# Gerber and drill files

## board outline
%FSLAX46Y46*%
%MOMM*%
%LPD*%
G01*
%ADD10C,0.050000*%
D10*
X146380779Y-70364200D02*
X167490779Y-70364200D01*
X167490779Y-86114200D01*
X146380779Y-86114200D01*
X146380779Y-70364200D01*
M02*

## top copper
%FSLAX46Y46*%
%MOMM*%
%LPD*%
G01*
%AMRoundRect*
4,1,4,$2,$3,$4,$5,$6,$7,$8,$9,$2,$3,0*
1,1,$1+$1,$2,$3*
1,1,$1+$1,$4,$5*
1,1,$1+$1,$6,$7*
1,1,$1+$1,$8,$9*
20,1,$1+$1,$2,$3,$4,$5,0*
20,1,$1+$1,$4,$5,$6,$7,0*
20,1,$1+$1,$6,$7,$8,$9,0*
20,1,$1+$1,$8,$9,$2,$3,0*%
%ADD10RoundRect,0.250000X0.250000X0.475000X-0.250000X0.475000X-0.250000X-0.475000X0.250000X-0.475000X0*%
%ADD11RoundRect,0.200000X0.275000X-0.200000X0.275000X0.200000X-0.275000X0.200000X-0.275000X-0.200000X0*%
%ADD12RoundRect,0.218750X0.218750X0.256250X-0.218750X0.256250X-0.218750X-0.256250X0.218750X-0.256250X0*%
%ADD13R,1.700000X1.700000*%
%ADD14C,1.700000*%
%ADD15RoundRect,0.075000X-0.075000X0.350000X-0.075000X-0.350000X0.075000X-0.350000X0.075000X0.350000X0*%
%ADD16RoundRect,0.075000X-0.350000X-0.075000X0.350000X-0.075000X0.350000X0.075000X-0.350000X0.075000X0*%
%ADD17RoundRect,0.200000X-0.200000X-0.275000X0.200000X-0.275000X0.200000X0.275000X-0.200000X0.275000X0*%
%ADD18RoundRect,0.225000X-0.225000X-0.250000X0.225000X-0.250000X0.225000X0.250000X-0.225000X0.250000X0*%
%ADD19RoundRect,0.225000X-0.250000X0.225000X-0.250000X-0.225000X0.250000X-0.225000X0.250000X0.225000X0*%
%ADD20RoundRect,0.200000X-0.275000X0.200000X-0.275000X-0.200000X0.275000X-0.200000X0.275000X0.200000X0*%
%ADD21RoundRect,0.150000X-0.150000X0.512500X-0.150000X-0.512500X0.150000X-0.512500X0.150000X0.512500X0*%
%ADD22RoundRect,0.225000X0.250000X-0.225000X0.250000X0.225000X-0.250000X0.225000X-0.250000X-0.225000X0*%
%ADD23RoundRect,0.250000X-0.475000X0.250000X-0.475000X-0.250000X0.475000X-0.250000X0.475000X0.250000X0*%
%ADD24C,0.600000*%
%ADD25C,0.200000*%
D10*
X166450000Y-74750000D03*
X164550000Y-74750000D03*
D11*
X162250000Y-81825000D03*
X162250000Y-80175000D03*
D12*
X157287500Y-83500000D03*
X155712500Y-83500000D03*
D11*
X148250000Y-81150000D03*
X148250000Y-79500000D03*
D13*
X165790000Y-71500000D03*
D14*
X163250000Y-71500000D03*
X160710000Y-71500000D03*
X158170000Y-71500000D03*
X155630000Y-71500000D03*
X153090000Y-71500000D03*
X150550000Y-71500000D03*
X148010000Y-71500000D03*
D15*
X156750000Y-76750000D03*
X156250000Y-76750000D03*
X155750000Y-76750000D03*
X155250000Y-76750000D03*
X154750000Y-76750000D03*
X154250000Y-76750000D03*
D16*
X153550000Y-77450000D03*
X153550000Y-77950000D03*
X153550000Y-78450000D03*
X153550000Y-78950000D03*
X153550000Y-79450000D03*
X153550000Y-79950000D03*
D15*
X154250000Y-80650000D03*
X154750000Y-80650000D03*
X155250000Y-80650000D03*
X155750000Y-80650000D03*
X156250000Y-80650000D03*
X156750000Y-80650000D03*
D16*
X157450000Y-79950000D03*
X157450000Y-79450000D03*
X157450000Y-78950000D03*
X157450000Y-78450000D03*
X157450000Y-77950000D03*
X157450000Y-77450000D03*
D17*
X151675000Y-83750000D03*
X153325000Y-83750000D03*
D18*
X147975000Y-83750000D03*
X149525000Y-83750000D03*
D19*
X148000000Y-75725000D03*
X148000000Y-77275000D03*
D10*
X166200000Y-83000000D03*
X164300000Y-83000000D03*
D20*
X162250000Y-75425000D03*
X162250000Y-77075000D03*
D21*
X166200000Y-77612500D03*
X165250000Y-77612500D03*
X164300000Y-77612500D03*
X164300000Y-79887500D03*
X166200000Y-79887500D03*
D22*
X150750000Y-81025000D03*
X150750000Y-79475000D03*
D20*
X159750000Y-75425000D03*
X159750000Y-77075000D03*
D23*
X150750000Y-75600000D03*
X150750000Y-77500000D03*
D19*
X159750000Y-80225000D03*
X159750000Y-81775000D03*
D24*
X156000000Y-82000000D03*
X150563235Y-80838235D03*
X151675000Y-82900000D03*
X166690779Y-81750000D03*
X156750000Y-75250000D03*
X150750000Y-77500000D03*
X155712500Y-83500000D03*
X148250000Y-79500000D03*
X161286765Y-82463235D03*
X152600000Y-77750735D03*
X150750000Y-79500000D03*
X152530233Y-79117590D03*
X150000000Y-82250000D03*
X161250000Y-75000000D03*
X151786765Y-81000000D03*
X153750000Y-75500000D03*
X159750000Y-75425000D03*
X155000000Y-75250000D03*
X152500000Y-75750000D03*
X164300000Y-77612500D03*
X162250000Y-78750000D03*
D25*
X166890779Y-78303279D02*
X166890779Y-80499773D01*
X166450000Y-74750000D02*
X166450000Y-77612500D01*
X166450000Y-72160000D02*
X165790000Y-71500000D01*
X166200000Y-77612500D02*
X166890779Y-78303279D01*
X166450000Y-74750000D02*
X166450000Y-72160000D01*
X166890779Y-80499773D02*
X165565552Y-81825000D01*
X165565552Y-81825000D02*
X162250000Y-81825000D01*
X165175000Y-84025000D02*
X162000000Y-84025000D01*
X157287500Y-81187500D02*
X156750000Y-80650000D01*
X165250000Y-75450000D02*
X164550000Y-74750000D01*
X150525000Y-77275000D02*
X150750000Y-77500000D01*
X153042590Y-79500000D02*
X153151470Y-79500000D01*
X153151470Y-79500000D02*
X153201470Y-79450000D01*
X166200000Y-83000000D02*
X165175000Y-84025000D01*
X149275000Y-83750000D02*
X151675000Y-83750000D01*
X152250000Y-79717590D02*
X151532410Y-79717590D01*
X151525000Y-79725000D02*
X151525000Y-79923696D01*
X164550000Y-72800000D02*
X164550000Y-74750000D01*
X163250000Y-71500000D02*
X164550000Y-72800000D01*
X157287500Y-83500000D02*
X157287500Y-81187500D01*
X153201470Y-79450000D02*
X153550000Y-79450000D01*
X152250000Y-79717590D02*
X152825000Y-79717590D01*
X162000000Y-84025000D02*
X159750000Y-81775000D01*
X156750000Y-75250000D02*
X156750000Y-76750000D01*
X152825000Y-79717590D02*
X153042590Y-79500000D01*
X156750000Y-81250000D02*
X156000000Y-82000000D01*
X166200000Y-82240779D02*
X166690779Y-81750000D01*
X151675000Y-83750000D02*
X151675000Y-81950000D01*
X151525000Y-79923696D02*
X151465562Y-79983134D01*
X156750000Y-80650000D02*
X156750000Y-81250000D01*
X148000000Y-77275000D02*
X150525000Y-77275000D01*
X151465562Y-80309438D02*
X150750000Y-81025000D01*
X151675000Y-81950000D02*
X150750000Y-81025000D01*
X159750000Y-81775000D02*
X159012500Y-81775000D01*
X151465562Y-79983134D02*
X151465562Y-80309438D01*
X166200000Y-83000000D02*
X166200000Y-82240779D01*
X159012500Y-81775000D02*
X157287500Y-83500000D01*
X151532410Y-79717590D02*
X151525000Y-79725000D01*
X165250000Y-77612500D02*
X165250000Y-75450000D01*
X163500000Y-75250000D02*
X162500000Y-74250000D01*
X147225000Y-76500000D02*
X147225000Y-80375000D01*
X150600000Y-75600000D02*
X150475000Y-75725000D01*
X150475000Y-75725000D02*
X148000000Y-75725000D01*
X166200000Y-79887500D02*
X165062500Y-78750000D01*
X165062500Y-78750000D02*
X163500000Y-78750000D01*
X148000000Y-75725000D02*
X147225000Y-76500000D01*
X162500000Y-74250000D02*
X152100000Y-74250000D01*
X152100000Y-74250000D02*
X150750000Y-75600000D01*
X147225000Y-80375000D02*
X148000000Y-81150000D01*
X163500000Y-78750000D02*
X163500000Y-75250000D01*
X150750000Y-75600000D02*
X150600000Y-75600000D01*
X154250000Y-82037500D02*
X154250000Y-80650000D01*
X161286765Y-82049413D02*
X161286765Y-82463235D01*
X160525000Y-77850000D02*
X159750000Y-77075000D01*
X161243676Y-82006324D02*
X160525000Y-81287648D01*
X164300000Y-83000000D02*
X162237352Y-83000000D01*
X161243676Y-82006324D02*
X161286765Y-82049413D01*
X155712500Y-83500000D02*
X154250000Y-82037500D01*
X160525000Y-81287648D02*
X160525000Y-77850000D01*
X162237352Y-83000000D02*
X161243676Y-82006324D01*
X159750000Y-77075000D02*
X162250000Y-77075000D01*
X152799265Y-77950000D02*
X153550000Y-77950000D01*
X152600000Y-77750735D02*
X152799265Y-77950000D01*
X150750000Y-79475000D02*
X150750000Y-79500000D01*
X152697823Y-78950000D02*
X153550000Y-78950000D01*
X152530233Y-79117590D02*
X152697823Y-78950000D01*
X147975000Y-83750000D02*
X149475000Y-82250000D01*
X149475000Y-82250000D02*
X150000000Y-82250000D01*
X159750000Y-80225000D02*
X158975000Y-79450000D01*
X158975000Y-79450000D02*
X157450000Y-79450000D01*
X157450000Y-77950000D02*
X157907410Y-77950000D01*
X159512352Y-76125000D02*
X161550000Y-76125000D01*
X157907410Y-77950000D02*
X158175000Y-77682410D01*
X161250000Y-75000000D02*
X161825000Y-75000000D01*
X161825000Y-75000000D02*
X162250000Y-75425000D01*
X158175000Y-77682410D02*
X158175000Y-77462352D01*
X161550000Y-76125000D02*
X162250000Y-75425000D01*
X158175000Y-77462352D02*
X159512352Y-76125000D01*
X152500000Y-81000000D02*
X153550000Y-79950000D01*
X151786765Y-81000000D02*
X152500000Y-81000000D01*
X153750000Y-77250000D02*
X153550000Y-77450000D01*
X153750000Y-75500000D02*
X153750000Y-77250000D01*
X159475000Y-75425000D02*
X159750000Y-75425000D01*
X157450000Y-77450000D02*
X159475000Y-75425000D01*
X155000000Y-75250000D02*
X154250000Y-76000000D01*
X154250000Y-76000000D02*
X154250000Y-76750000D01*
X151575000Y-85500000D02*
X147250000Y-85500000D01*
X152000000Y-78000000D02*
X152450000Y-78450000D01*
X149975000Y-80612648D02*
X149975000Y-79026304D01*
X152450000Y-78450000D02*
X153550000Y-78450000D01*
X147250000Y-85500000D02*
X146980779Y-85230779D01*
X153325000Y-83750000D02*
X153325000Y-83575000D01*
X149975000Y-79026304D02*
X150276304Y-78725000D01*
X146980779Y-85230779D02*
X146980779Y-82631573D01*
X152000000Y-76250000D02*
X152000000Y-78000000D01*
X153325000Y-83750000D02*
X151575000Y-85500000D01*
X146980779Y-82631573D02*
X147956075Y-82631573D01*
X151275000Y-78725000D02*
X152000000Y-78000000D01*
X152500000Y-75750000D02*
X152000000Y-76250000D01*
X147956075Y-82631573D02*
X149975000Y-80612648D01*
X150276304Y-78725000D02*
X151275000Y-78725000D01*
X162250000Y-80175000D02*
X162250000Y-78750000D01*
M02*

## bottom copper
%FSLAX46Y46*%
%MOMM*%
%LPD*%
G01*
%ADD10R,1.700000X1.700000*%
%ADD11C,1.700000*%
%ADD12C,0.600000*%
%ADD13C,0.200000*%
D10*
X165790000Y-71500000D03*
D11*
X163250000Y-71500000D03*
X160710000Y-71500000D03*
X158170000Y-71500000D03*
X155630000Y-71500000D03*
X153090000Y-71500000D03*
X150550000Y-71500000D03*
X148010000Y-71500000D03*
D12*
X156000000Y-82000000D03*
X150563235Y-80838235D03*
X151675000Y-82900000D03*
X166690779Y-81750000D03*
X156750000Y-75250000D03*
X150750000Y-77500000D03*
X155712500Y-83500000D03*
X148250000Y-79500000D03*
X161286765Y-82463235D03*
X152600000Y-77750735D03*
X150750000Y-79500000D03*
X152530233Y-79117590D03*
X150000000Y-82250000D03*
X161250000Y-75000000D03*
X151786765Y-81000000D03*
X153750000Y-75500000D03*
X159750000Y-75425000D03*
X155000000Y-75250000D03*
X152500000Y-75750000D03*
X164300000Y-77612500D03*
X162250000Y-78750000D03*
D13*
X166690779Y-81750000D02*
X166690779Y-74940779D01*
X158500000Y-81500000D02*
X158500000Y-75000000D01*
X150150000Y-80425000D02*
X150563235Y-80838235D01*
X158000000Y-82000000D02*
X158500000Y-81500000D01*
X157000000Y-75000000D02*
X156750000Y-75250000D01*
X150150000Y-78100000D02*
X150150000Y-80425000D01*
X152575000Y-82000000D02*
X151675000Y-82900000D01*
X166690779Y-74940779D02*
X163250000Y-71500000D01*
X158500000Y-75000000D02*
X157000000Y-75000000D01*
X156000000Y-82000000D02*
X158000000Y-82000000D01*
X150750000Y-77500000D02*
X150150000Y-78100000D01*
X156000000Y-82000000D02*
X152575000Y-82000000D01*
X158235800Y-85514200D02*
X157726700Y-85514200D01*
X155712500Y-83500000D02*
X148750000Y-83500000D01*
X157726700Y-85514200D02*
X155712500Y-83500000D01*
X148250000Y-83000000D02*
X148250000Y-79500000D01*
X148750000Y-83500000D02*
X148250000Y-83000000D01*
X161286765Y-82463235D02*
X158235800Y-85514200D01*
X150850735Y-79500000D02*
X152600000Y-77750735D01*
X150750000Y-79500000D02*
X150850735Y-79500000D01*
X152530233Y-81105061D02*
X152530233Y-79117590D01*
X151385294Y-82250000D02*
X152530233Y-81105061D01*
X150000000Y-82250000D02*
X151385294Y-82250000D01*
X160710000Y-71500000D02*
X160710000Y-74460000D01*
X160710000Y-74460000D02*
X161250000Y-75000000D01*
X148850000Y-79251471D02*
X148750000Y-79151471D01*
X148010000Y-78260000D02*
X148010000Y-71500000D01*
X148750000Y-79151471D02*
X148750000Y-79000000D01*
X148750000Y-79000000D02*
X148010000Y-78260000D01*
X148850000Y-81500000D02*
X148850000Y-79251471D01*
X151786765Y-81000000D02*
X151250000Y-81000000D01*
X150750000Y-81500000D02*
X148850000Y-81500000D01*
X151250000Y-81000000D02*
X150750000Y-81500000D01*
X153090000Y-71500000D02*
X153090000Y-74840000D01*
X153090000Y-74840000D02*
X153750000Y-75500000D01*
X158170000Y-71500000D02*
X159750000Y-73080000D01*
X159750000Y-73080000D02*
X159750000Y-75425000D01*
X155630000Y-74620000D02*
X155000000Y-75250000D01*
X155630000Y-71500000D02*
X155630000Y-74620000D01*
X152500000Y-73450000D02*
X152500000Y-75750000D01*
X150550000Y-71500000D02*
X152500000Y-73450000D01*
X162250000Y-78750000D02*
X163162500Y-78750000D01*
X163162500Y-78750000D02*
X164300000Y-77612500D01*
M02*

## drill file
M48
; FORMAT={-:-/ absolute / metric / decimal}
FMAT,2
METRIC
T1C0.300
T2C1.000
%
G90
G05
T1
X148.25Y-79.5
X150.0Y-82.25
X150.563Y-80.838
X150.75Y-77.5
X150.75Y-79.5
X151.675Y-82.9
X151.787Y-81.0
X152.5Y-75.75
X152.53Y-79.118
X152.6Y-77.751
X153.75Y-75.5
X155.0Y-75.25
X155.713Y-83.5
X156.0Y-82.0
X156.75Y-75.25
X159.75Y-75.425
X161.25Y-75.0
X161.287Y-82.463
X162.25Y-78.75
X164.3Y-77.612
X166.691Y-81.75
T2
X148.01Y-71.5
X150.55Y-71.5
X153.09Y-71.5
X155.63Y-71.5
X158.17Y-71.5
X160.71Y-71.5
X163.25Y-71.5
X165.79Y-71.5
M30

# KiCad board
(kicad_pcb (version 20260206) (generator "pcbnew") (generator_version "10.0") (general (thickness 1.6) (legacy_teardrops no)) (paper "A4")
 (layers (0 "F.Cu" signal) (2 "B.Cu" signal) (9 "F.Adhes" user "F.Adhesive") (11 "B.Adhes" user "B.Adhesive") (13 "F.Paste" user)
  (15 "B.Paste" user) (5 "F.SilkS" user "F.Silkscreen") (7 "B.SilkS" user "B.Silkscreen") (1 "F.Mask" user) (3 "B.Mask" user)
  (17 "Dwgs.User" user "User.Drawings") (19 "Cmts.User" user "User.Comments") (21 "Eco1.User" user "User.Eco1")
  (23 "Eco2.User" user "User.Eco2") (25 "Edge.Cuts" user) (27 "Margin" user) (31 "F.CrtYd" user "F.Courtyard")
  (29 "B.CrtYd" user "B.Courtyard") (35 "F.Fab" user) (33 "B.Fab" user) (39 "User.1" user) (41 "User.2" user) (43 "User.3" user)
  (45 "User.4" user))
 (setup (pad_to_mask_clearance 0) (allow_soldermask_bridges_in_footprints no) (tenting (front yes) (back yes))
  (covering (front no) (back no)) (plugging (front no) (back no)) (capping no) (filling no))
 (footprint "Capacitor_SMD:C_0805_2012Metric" (layer "F.Cu") (at 165.5 74.75 180)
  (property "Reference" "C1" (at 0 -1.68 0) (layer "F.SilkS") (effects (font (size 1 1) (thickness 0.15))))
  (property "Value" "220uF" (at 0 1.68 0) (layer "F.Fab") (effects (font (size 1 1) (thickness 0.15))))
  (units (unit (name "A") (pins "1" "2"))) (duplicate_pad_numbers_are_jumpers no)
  (pad "1" smd roundrect (at -0.95 0 180) (size 1 1.45) (layers "F.Cu" "F.Mask" "F.Paste") (roundrect_rratio 0.25) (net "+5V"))
  (pad "2" smd roundrect (at 0.95 0 180) (size 1 1.45) (layers "F.Cu" "F.Mask" "F.Paste") (roundrect_rratio 0.25) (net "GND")))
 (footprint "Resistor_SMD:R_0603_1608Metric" (layer "F.Cu") (at 162.25 81 90)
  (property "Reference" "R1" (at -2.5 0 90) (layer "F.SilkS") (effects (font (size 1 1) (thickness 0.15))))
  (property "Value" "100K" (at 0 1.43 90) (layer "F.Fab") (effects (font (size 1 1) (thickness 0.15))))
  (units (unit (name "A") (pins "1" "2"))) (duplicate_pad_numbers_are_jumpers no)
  (pad "1" smd roundrect (at -0.825 0 90) (size 0.8 0.95) (layers "F.Cu" "F.Mask" "F.Paste") (roundrect_rratio 0.25) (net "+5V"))
  (pad "2" smd roundrect (at 0.825 0 90) (size 0.8 0.95) (layers "F.Cu" "F.Mask" "F.Paste") (roundrect_rratio 0.25) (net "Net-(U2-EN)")))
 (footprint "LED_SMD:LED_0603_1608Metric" (layer "F.Cu") (at 156.5 83.5 180)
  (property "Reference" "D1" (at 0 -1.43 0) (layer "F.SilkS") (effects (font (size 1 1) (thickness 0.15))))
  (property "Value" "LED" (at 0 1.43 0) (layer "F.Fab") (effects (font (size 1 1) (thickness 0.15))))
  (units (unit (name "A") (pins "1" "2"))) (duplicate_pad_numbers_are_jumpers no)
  (pad "1" smd roundrect (at -0.7875 0 180) (size 0.875 0.95) (layers "F.Cu" "F.Mask" "F.Paste") (roundrect_rratio 0.25) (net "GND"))
  (pad "2" smd roundrect (at 0.7875 0 180) (size 0.875 0.95) (layers "F.Cu" "F.Mask" "F.Paste") (roundrect_rratio 0.25) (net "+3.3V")))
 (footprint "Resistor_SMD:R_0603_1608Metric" (layer "F.Cu") (at 148.25 80.325 90)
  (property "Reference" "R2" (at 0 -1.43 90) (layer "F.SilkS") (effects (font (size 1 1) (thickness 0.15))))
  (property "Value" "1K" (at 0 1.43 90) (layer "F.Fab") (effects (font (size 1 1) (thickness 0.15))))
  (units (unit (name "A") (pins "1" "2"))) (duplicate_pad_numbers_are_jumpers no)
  (pad "1" smd roundrect (at -0.825 0 90) (size 0.8 0.95) (layers "F.Cu" "F.Mask" "F.Paste") (roundrect_rratio 0.25) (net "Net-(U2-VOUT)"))
  (pad "2" smd roundrect (at 0.825 0 90) (size 0.8 0.95) (layers "F.Cu" "F.Mask" "F.Paste") (roundrect_rratio 0.25) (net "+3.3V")))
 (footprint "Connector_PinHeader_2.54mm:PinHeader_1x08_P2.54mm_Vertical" (layer "F.Cu") (at 165.79 71.5 -90)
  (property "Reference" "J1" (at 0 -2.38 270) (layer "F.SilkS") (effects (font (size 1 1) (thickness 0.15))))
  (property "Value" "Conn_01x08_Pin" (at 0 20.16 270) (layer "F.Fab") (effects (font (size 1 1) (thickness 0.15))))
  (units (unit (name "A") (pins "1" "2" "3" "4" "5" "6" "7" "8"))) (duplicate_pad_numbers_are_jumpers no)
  (pad "1" thru_hole rect (at 0 0 270) (size 1.7 1.7) (drill 1) (layers "*.Cu" "*.Mask") (remove_unused_layers no) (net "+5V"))
  (pad "2" thru_hole circle (at 0 2.54 270) (size 1.7 1.7) (drill 1) (layers "*.Cu" "*.Mask") (remove_unused_layers no) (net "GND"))
  (pad "3" thru_hole circle (at 0 5.08 270) (size 1.7 1.7) (drill 1) (layers "*.Cu" "*.Mask") (remove_unused_layers no) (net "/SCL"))
  (pad "4" thru_hole circle (at 0 7.62 270) (size 1.7 1.7) (drill 1) (layers "*.Cu" "*.Mask") (remove_unused_layers no) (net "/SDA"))
  (pad "5" thru_hole circle (at 0 10.16 270) (size 1.7 1.7) (drill 1) (layers "*.Cu" "*.Mask") (remove_unused_layers no) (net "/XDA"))
  (pad "6" thru_hole circle (at 0 12.7 270) (size 1.7 1.7) (drill 1) (layers "*.Cu" "*.Mask") (remove_unused_layers no) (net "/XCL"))
  (pad "7" thru_hole circle (at 0 15.24 270) (size 1.7 1.7) (drill 1) (layers "*.Cu" "*.Mask") (remove_unused_layers no) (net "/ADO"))
  (pad "8" thru_hole circle (at 0 17.78 270) (size 1.7 1.7) (drill 1) (layers "*.Cu" "*.Mask") (remove_unused_layers no) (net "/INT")))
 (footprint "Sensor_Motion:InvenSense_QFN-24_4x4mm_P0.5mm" (layer "F.Cu") (at 155.5 78.7 -90)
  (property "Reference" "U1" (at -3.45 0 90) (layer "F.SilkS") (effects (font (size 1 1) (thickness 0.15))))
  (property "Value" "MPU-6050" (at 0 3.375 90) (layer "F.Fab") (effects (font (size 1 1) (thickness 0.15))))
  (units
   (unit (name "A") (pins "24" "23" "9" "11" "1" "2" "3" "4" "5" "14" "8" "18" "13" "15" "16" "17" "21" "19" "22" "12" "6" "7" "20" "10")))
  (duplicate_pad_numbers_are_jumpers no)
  (pad "1" smd roundrect (at -1.95 -1.25 270) (size 0.85 0.3) (layers "F.Cu" "F.Mask" "F.Paste") (roundrect_rratio 0.25) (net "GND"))
  (pad "2" smd roundrect (at -1.95 -0.75 270) (size 0.85 0.3) (layers "F.Cu" "F.Mask" "F.Paste") (roundrect_rratio 0.25)
   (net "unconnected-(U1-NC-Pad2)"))
  (pad "3" smd roundrect (at -1.95 -0.25 270) (size 0.85 0.3) (layers "F.Cu" "F.Mask" "F.Paste") (roundrect_rratio 0.25)
   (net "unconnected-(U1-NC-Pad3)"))
  (pad "4" smd roundrect (at -1.95 0.25 270) (size 0.85 0.3) (layers "F.Cu" "F.Mask" "F.Paste") (roundrect_rratio 0.25)
   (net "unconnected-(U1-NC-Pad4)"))
  (pad "5" smd roundrect (at -1.95 0.75 270) (size 0.85 0.3) (layers "F.Cu" "F.Mask" "F.Paste") (roundrect_rratio 0.25)
   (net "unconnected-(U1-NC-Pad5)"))
  (pad "6" smd roundrect (at -1.95 1.25 270) (size 0.85 0.3) (layers "F.Cu" "F.Mask" "F.Paste") (roundrect_rratio 0.25) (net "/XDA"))
  (pad "7" smd roundrect (at -1.25 1.95) (size 0.85 0.3) (layers "F.Cu" "F.Mask" "F.Paste") (roundrect_rratio 0.25) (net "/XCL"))
  (pad "8" smd roundrect (at -0.75 1.95) (size 0.85 0.3) (layers "F.Cu" "F.Mask" "F.Paste") (roundrect_rratio 0.25) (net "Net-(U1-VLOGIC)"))
  (pad "9" smd roundrect (at -0.25 1.95) (size 0.85 0.3) (layers "F.Cu" "F.Mask" "F.Paste") (roundrect_rratio 0.25) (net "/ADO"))
  (pad "10" smd roundrect (at 0.25 1.95) (size 0.85 0.3) (layers "F.Cu" "F.Mask" "F.Paste") (roundrect_rratio 0.25) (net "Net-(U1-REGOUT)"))
  (pad "11" smd roundrect (at 0.75 1.95) (size 0.85 0.3) (layers "F.Cu" "F.Mask" "F.Paste") (roundrect_rratio 0.25) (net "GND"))
  (pad "12" smd roundrect (at 1.25 1.95) (size 0.85 0.3) (layers "F.Cu" "F.Mask" "F.Paste") (roundrect_rratio 0.25) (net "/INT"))
  (pad "13" smd roundrect (at 1.95 1.25 270) (size 0.85 0.3) (layers "F.Cu" "F.Mask" "F.Paste") (roundrect_rratio 0.25) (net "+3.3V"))
  (pad "14" smd roundrect (at 1.95 0.75 270) (size 0.85 0.3) (layers "F.Cu" "F.Mask" "F.Paste") (roundrect_rratio 0.25)
   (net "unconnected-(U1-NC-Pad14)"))
  (pad "15" smd roundrect (at 1.95 0.25 270) (size 0.85 0.3) (layers "F.Cu" "F.Mask" "F.Paste") (roundrect_rratio 0.25)
   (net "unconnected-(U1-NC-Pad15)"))
  (pad "16" smd roundrect (at 1.95 -0.25 270) (size 0.85 0.3) (layers "F.Cu" "F.Mask" "F.Paste") (roundrect_rratio 0.25)
   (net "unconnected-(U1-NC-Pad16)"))
  (pad "17" smd roundrect (at 1.95 -0.75 270) (size 0.85 0.3) (layers "F.Cu" "F.Mask" "F.Paste") (roundrect_rratio 0.25)
   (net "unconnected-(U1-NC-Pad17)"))
  (pad "18" smd roundrect (at 1.95 -1.25 270) (size 0.85 0.3) (layers "F.Cu" "F.Mask" "F.Paste") (roundrect_rratio 0.25) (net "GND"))
  (pad "19" smd roundrect (at 1.25 -1.95) (size 0.85 0.3) (layers "F.Cu" "F.Mask" "F.Paste") (roundrect_rratio 0.25)
   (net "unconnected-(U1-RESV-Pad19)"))
  (pad "20" smd roundrect (at 0.75 -1.95) (size 0.85 0.3) (layers "F.Cu" "F.Mask" "F.Paste") (roundrect_rratio 0.25) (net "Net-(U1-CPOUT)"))
  (pad "21" smd roundrect (at 0.25 -1.95) (size 0.85 0.3) (layers "F.Cu" "F.Mask" "F.Paste") (roundrect_rratio 0.25)
   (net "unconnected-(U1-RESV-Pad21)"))
  (pad "22" smd roundrect (at -0.25 -1.95) (size 0.85 0.3) (layers "F.Cu" "F.Mask" "F.Paste") (roundrect_rratio 0.25)
   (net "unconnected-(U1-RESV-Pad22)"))
  (pad "23" smd roundrect (at -0.75 -1.95) (size 0.85 0.3) (layers "F.Cu" "F.Mask" "F.Paste") (roundrect_rratio 0.25) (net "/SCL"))
  (pad "24" smd roundrect (at -1.25 -1.95) (size 0.85 0.3) (layers "F.Cu" "F.Mask" "F.Paste") (roundrect_rratio 0.25) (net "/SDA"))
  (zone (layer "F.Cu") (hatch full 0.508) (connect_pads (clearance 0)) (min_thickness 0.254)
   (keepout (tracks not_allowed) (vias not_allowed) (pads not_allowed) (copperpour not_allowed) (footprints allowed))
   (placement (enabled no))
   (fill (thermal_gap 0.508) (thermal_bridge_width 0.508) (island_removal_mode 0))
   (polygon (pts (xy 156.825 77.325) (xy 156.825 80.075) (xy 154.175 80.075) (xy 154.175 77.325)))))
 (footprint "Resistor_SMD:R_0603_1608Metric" (layer "F.Cu") (at 152.5 83.75)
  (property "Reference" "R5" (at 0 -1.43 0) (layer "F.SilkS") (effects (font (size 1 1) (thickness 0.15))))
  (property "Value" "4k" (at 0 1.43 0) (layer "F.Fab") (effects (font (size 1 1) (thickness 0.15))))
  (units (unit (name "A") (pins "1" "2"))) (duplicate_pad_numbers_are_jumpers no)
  (pad "1" smd roundrect (at -0.825 0) (size 0.8 0.95) (layers "F.Cu" "F.Mask" "F.Paste") (roundrect_rratio 0.25) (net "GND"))
  (pad "2" smd roundrect (at 0.825 0) (size 0.8 0.95) (layers "F.Cu" "F.Mask" "F.Paste") (roundrect_rratio 0.25) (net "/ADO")))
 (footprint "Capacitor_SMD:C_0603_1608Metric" (layer "F.Cu") (at 148.75 83.75)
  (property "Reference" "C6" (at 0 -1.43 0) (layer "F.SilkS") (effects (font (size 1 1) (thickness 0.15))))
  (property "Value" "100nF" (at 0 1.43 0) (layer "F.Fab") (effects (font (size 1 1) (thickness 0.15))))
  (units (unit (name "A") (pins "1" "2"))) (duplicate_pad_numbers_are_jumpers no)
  (pad "1" smd roundrect (at -0.775 0) (size 0.9 0.95) (layers "F.Cu" "F.Mask" "F.Paste") (roundrect_rratio 0.25) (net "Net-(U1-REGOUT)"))
  (pad "2" smd roundrect (at 0.775 0) (size 0.9 0.95) (layers "F.Cu" "F.Mask" "F.Paste") (roundrect_rratio 0.25) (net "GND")))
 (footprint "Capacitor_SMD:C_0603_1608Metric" (layer "F.Cu") (at 148 76.5 -90)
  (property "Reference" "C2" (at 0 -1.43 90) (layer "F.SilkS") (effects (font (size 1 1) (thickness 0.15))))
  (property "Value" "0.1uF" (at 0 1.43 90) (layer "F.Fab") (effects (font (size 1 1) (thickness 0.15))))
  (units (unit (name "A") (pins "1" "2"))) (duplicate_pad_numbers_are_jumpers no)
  (pad "1" smd roundrect (at -0.775 0 270) (size 0.9 0.95) (layers "F.Cu" "F.Mask" "F.Paste") (roundrect_rratio 0.25) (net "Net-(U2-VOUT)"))
  (pad "2" smd roundrect (at 0.775 0 270) (size 0.9 0.95) (layers "F.Cu" "F.Mask" "F.Paste") (roundrect_rratio 0.25) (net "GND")))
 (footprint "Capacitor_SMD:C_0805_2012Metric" (layer "F.Cu") (at 165.25 83 180)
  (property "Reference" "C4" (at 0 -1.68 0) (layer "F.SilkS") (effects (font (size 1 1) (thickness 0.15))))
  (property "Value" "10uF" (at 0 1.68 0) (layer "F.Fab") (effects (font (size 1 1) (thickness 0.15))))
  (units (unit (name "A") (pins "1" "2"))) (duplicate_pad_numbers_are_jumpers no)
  (pad "1" smd roundrect (at -0.95 0 180) (size 1 1.45) (layers "F.Cu" "F.Mask" "F.Paste") (roundrect_rratio 0.25) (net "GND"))
  (pad "2" smd roundrect (at 0.95 0 180) (size 1 1.45) (layers "F.Cu" "F.Mask" "F.Paste") (roundrect_rratio 0.25) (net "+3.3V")))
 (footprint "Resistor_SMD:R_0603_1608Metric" (layer "F.Cu") (at 162.25 76.25 -90)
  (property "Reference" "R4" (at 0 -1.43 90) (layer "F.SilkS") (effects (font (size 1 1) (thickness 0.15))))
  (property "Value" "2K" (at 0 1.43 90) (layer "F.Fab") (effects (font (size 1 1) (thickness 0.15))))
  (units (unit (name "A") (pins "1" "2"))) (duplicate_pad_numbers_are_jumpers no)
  (pad "1" smd roundrect (at -0.825 0 270) (size 0.8 0.95) (layers "F.Cu" "F.Mask" "F.Paste") (roundrect_rratio 0.25) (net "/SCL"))
  (pad "2" smd roundrect (at 0.825 0 270) (size 0.8 0.95) (layers "F.Cu" "F.Mask" "F.Paste") (roundrect_rratio 0.25) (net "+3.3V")))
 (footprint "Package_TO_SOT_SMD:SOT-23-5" (layer "F.Cu") (at 165.25 78.75 -90)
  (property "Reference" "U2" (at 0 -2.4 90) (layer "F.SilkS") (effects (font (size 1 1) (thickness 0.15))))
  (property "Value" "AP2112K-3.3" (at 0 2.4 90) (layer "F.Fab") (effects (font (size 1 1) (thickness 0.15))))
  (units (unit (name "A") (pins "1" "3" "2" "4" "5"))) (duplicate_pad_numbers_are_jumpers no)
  (pad "1" smd roundrect (at -1.1375 -0.95 270) (size 1.325 0.6) (layers "F.Cu" "F.Mask" "F.Paste") (roundrect_rratio 0.25) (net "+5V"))
  (pad "2" smd roundrect (at -1.1375 0 270) (size 1.325 0.6) (layers "F.Cu" "F.Mask" "F.Paste") (roundrect_rratio 0.25) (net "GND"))
  (pad "3" smd roundrect (at -1.1375 0.95 270) (size 1.325 0.6) (layers "F.Cu" "F.Mask" "F.Paste") (roundrect_rratio 0.25)
   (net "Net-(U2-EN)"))
  (pad "4" smd roundrect (at 1.1375 0.95 270) (size 1.325 0.6) (layers "F.Cu" "F.Mask" "F.Paste") (roundrect_rratio 0.25)
   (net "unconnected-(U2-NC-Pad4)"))
  (pad "5" smd roundrect (at 1.1375 -0.95 270) (size 1.325 0.6) (layers "F.Cu" "F.Mask" "F.Paste") (roundrect_rratio 0.25)
   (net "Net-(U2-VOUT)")))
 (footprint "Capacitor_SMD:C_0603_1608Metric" (layer "F.Cu") (at 150.75 80.25 90)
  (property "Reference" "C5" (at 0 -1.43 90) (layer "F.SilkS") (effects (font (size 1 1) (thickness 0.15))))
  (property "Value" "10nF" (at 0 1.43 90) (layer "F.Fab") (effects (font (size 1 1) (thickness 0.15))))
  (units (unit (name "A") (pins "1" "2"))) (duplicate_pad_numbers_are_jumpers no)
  (pad "1" smd roundrect (at -0.775 0 90) (size 0.9 0.95) (layers "F.Cu" "F.Mask" "F.Paste") (roundrect_rratio 0.25) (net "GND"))
  (pad "2" smd roundrect (at 0.775 0 90) (size 0.9 0.95) (layers "F.Cu" "F.Mask" "F.Paste") (roundrect_rratio 0.25) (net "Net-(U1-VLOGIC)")))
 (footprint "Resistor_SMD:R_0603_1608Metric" (layer "F.Cu") (at 159.75 76.25 -90)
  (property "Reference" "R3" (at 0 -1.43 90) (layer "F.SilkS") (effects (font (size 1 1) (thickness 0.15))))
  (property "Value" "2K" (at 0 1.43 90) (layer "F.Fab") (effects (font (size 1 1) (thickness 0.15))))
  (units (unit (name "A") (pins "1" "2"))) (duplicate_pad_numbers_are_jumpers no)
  (pad "1" smd roundrect (at -0.825 0 270) (size 0.8 0.95) (layers "F.Cu" "F.Mask" "F.Paste") (roundrect_rratio 0.25) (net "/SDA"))
  (pad "2" smd roundrect (at 0.825 0 270) (size 0.8 0.95) (layers "F.Cu" "F.Mask" "F.Paste") (roundrect_rratio 0.25) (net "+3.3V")))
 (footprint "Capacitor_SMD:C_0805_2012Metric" (layer "F.Cu") (at 150.75 76.55 -90)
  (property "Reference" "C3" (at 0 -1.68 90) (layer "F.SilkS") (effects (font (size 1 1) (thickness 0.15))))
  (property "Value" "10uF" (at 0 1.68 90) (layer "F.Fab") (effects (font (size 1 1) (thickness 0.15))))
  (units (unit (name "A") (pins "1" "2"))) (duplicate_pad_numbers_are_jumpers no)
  (pad "1" smd roundrect (at -0.95 0 270) (size 1 1.45) (layers "F.Cu" "F.Mask" "F.Paste") (roundrect_rratio 0.25) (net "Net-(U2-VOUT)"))
  (pad "2" smd roundrect (at 0.95 0 270) (size 1 1.45) (layers "F.Cu" "F.Mask" "F.Paste") (roundrect_rratio 0.25) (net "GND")))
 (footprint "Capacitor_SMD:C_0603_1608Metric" (layer "F.Cu") (at 159.75 81 -90)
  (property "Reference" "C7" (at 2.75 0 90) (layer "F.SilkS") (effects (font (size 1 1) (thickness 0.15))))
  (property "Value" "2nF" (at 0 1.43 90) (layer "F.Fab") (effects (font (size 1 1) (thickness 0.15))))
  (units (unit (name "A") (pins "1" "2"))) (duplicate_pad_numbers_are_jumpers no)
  (pad "1" smd roundrect (at -0.775 0 270) (size 0.9 0.95) (layers "F.Cu" "F.Mask" "F.Paste") (roundrect_rratio 0.25) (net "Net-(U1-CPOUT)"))
  (pad "2" smd roundrect (at 0.775 0 270) (size 0.9 0.95) (layers "F.Cu" "F.Mask" "F.Paste") (roundrect_rratio 0.25) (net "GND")))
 (gr_rect (start 146.380779 70.3642) (end 167.490779 86.1142) (stroke (width 0.05) (type solid)) (fill no) (layer "Edge.Cuts"))
 (segment (start 166.890779 78.303279) (end 166.890779 80.499773) (width 0.2) (layer "F.Cu") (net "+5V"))
 (segment (start 166.45 74.75) (end 166.45 77.6125) (width 0.2) (layer "F.Cu") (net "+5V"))
 (segment (start 166.45 72.16) (end 165.79 71.5) (width 0.2) (layer "F.Cu") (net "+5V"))
 (segment (start 166.2 77.6125) (end 166.890779 78.303279) (width 0.2) (layer "F.Cu") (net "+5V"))
 (segment (start 166.45 74.75) (end 166.45 72.16) (width 0.2) (layer "F.Cu") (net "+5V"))
 (segment (start 166.890779 80.499773) (end 165.565552 81.825) (width 0.2) (layer "F.Cu") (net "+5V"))
 (segment (start 165.565552 81.825) (end 162.25 81.825) (width 0.2) (layer "F.Cu") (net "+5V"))
 (segment (start 165.175 84.025) (end 162 84.025) (width 0.2) (layer "F.Cu") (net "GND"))
 (segment (start 157.2875 81.1875) (end 156.75 80.65) (width 0.2) (layer "F.Cu") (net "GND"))
 (segment (start 165.25 75.45) (end 164.55 74.75) (width 0.2) (layer "F.Cu") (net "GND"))
 (segment (start 150.525 77.275) (end 150.75 77.5) (width 0.2) (layer "F.Cu") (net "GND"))
 (segment (start 153.04259 79.5) (end 153.15147 79.5) (width 0.2) (layer "F.Cu") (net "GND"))
 (segment (start 153.15147 79.5) (end 153.20147 79.45) (width 0.2) (layer "F.Cu") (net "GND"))
 (segment (start 166.2 83) (end 165.175 84.025) (width 0.2) (layer "F.Cu") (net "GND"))
 (segment (start 149.275 83.75) (end 151.675 83.75) (width 0.2) (layer "F.Cu") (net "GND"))
 (segment (start 152.25 79.71759) (end 151.53241 79.71759) (width 0.2) (layer "F.Cu") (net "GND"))
 (segment (start 151.525 79.725) (end 151.525 79.923696) (width 0.2) (layer "F.Cu") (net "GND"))
 (segment (start 164.55 72.8) (end 164.55 74.75) (width 0.2) (layer "F.Cu") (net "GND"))
 (segment (start 163.25 71.5) (end 164.55 72.8) (width 0.2) (layer "F.Cu") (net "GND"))
 (segment (start 157.2875 83.5) (end 157.2875 81.1875) (width 0.2) (layer "F.Cu") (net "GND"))
 (segment (start 153.20147 79.45) (end 153.55 79.45) (width 0.2) (layer "F.Cu") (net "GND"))
 (segment (start 152.25 79.71759) (end 152.825 79.71759) (width 0.2) (layer "F.Cu") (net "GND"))
 (segment (start 162 84.025) (end 159.75 81.775) (width 0.2) (layer "F.Cu") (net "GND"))
 (segment (start 156.75 75.25) (end 156.75 76.75) (width 0.2) (layer "F.Cu") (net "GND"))
 (segment (start 152.825 79.71759) (end 153.04259 79.5) (width 0.2) (layer "F.Cu") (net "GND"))
 (segment (start 156.75 81.25) (end 156 82) (width 0.2) (layer "F.Cu") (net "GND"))
 (segment (start 166.2 82.240779) (end 166.690779 81.75) (width 0.2) (layer "F.Cu") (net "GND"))
 (segment (start 151.675 83.75) (end 151.675 81.95) (width 0.2) (layer "F.Cu") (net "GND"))
 (segment (start 151.525 79.923696) (end 151.465562 79.983134) (width 0.2) (layer "F.Cu") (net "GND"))
 (segment (start 156.75 80.65) (end 156.75 81.25) (width 0.2) (layer "F.Cu") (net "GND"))
 (segment (start 148 77.275) (end 150.525 77.275) (width 0.2) (layer "F.Cu") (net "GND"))
 (segment (start 151.465562 80.309438) (end 150.75 81.025) (width 0.2) (layer "F.Cu") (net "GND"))
 (segment (start 151.675 81.95) (end 150.75 81.025) (width 0.2) (layer "F.Cu") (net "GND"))
 (segment (start 159.75 81.775) (end 159.0125 81.775) (width 0.2) (layer "F.Cu") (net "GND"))
 (segment (start 151.465562 79.983134) (end 151.465562 80.309438) (width 0.2) (layer "F.Cu") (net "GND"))
 (segment (start 166.2 83) (end 166.2 82.240779) (width 0.2) (layer "F.Cu") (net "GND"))
 (segment (start 159.0125 81.775) (end 157.2875 83.5) (width 0.2) (layer "F.Cu") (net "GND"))
 (segment (start 151.53241 79.71759) (end 151.525 79.725) (width 0.2) (layer "F.Cu") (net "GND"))
 (segment (start 165.25 77.6125) (end 165.25 75.45) (width 0.2) (layer "F.Cu") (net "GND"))
 (via (at 156 82) (size 0.6) (drill 0.3) (layers "F.Cu" "B.Cu") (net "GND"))
 (via (at 150.563235 80.838235) (size 0.6) (drill 0.3) (layers "F.Cu" "B.Cu") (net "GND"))
 (via (at 151.675 82.9) (size 0.6) (drill 0.3) (layers "F.Cu" "B.Cu") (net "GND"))
 (via (at 166.690779 81.75) (size 0.6) (drill 0.3) (layers "F.Cu" "B.Cu") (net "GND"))
 (via (at 156.75 75.25) (size 0.6) (drill 0.3) (layers "F.Cu" "B.Cu") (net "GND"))
 (via (at 150.75 77.5) (size 0.6) (drill 0.3) (layers "F.Cu" "B.Cu") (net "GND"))
 (segment (start 166.690779 81.75) (end 166.690779 74.940779) (width 0.2) (layer "B.Cu") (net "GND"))
 (segment (start 158.5 81.5) (end 158.5 75) (width 0.2) (layer "B.Cu") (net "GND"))
 (segment (start 150.15 80.425) (end 150.563235 80.838235) (width 0.2) (layer "B.Cu") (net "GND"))
 (segment (start 158 82) (end 158.5 81.5) (width 0.2) (layer "B.Cu") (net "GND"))
 (segment (start 157 75) (end 156.75 75.25) (width 0.2) (layer "B.Cu") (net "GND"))
 (segment (start 150.15 78.1) (end 150.15 80.425) (width 0.2) (layer "B.Cu") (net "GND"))
 (segment (start 152.575 82) (end 151.675 82.9) (width 0.2) (layer "B.Cu") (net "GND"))
 (segment (start 166.690779 74.940779) (end 163.25 71.5) (width 0.2) (layer "B.Cu") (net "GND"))
 (segment (start 158.5 75) (end 157 75) (width 0.2) (layer "B.Cu") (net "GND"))
 (segment (start 156 82) (end 158 82) (width 0.2) (layer "B.Cu") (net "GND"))
 (segment (start 150.75 77.5) (end 150.15 78.1) (width 0.2) (layer "B.Cu") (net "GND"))
 (segment (start 156 82) (end 152.575 82) (width 0.2) (layer "B.Cu") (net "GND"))
 (segment (start 163.5 75.25) (end 162.5 74.25) (width 0.2) (layer "F.Cu") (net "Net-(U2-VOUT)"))
 (segment (start 147.225 76.5) (end 147.225 80.375) (width 0.2) (layer "F.Cu") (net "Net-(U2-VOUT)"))
 (segment (start 150.6 75.6) (end 150.475 75.725) (width 0.2) (layer "F.Cu") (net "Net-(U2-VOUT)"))
 (segment (start 150.475 75.725) (end 148 75.725) (width 0.2) (layer "F.Cu") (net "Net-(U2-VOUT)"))
 (segment (start 166.2 79.8875) (end 165.0625 78.75) (width 0.2) (layer "F.Cu") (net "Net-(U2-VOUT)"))
 (segment (start 165.0625 78.75) (end 163.5 78.75) (width 0.2) (layer "F.Cu") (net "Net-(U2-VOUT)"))
 (segment (start 148 75.725) (end 147.225 76.5) (width 0.2) (layer "F.Cu") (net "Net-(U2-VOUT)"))
 (segment (start 162.5 74.25) (end 152.1 74.25) (width 0.2) (layer "F.Cu") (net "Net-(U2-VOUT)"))
 (segment (start 152.1 74.25) (end 150.75 75.6) (width 0.2) (layer "F.Cu") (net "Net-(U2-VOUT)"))
 (segment (start 147.225 80.375) (end 148 81.15) (width 0.2) (layer "F.Cu") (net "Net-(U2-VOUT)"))
 (segment (start 163.5 78.75) (end 163.5 75.25) (width 0.2) (layer "F.Cu") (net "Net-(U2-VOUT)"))
 (segment (start 150.75 75.6) (end 150.6 75.6) (width 0.2) (layer "F.Cu") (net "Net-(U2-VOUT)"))
 (segment (start 154.25 82.0375) (end 154.25 80.65) (width 0.2) (layer "F.Cu") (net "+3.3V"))
 (segment (start 161.286765 82.049413) (end 161.286765 82.463235) (width 0.2) (layer "F.Cu") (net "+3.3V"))
 (segment (start 160.525 77.85) (end 159.75 77.075) (width 0.2) (layer "F.Cu") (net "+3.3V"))
 (segment (start 161.243676 82.006324) (end 160.525 81.287648) (width 0.2) (layer "F.Cu") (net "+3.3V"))
 (segment (start 164.3 83) (end 162.237352 83) (width 0.2) (layer "F.Cu") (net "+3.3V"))
 (segment (start 161.243676 82.006324) (end 161.286765 82.049413) (width 0.2) (layer "F.Cu") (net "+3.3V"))
 (segment (start 155.7125 83.5) (end 154.25 82.0375) (width 0.2) (layer "F.Cu") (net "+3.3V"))
 (segment (start 160.525 81.287648) (end 160.525 77.85) (width 0.2) (layer "F.Cu") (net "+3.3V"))
 (segment (start 162.237352 83) (end 161.243676 82.006324) (width 0.2) (layer "F.Cu") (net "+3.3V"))
 (segment (start 159.75 77.075) (end 162.25 77.075) (width 0.2) (layer "F.Cu") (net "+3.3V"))
 (via (at 155.7125 83.5) (size 0.6) (drill 0.3) (layers "F.Cu" "B.Cu") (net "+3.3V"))
 (via (at 148.25 79.5) (size 0.6) (drill 0.3) (layers "F.Cu" "B.Cu") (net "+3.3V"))
 (via (at 161.286765 82.463235) (size 0.6) (drill 0.3) (layers "F.Cu" "B.Cu") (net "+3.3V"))
 (segment (start 158.2358 85.5142) (end 157.7267 85.5142) (width 0.2) (layer "B.Cu") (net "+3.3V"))
 (segment (start 155.7125 83.5) (end 148.75 83.5) (width 0.2) (layer "B.Cu") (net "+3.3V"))
 (segment (start 157.7267 85.5142) (end 155.7125 83.5) (width 0.2) (layer "B.Cu") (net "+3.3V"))
 (segment (start 148.25 83) (end 148.25 79.5) (width 0.2) (layer "B.Cu") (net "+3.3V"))
 (segment (start 148.75 83.5) (end 148.25 83) (width 0.2) (layer "B.Cu") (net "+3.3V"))
 (segment (start 161.286765 82.463235) (end 158.2358 85.5142) (width 0.2) (layer "B.Cu") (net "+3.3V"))
 (segment (start 152.799265 77.95) (end 153.55 77.95) (width 0.2) (layer "F.Cu") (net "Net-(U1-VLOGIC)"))
 (segment (start 152.6 77.750735) (end 152.799265 77.95) (width 0.2) (layer "F.Cu") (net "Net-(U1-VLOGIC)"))
 (segment (start 150.75 79.475) (end 150.75 79.5) (width 0.2) (layer "F.Cu") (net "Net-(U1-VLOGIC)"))
 (via (at 152.6 77.750735) (size 0.6) (drill 0.3) (layers "F.Cu" "B.Cu") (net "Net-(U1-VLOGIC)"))
 (via (at 150.75 79.5) (size 0.6) (drill 0.3) (layers "F.Cu" "B.Cu") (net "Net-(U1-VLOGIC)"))
 (segment (start 150.850735 79.5) (end 152.6 77.750735) (width 0.2) (layer "B.Cu") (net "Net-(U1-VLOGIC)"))
 (segment (start 150.75 79.5) (end 150.850735 79.5) (width 0.2) (layer "B.Cu") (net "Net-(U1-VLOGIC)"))
 (segment (start 152.697823 78.95) (end 153.55 78.95) (width 0.2) (layer "F.Cu") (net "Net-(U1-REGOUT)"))
 (segment (start 152.530233 79.11759) (end 152.697823 78.95) (width 0.2) (layer "F.Cu") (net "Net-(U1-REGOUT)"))
 (segment (start 147.975 83.75) (end 149.475 82.25) (width 0.2) (layer "F.Cu") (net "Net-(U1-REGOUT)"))
 (segment (start 149.475 82.25) (end 150 82.25) (width 0.2) (layer "F.Cu") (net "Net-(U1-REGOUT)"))
 (via (at 152.530233 79.11759) (size 0.6) (drill 0.3) (layers "F.Cu" "B.Cu") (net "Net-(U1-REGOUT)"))
 (via (at 150 82.25) (size 0.6) (drill 0.3) (layers "F.Cu" "B.Cu") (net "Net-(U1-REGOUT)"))
 (segment (start 152.530233 81.105061) (end 152.530233 79.11759) (width 0.2) (layer "B.Cu") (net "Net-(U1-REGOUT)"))
 (segment (start 151.385294 82.25) (end 152.530233 81.105061) (width 0.2) (layer "B.Cu") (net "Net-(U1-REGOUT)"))
 (segment (start 150 82.25) (end 151.385294 82.25) (width 0.2) (layer "B.Cu") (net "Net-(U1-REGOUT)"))
 (segment (start 159.75 80.225) (end 158.975 79.45) (width 0.2) (layer "F.Cu") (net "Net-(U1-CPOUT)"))
 (segment (start 158.975 79.45) (end 157.45 79.45) (width 0.2) (layer "F.Cu") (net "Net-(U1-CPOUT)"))
 (segment (start 157.45 77.95) (end 157.90741 77.95) (width 0.2) (layer "F.Cu") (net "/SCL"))
 (segment (start 159.512352 76.125) (end 161.55 76.125) (width 0.2) (layer "F.Cu") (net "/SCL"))
 (segment (start 157.90741 77.95) (end 158.175 77.68241) (width 0.2) (layer "F.Cu") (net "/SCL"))
 (segment (start 161.25 75) (end 161.825 75) (width 0.2) (layer "F.Cu") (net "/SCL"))
 (segment (start 161.825 75) (end 162.25 75.425) (width 0.2) (layer "F.Cu") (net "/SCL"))
 (segment (start 158.175 77.68241) (end 158.175 77.462352) (width 0.2) (layer "F.Cu") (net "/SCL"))
 (segment (start 161.55 76.125) (end 162.25 75.425) (width 0.2) (layer "F.Cu") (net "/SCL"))
 (segment (start 158.175 77.462352) (end 159.512352 76.125) (width 0.2) (layer "F.Cu") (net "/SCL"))
 (via (at 161.25 75) (size 0.6) (drill 0.3) (layers "F.Cu" "B.Cu") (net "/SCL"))
 (segment (start 160.71 71.5) (end 160.71 74.46) (width 0.2) (layer "B.Cu") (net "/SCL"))
 (segment (start 160.71 74.46) (end 161.25 75) (width 0.2) (layer "B.Cu") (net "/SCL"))
 (segment (start 152.5 81) (end 153.55 79.95) (width 0.2) (layer "F.Cu") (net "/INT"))
 (segment (start 151.786765 81) (end 152.5 81) (width 0.2) (layer "F.Cu") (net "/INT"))
 (via (at 151.786765 81) (size 0.6) (drill 0.3) (layers "F.Cu" "B.Cu") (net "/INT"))
 (segment (start 148.85 79.251471) (end 148.75 79.151471) (width 0.2) (layer "B.Cu") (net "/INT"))
 (segment (start 148.01 78.26) (end 148.01 71.5) (width 0.2) (layer "B.Cu") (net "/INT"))
 (segment (start 148.75 79.151471) (end 148.75 79) (width 0.2) (layer "B.Cu") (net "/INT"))
 (segment (start 148.75 79) (end 148.01 78.26) (width 0.2) (layer "B.Cu") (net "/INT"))
 (segment (start 148.85 81.5) (end 148.85 79.251471) (width 0.2) (layer "B.Cu") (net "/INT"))
 (segment (start 151.786765 81) (end 151.25 81) (width 0.2) (layer "B.Cu") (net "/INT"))
 (segment (start 150.75 81.5) (end 148.85 81.5) (width 0.2) (layer "B.Cu") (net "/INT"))
 (segment (start 151.25 81) (end 150.75 81.5) (width 0.2) (layer "B.Cu") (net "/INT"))
 (segment (start 153.75 77.25) (end 153.55 77.45) (width 0.2) (layer "F.Cu") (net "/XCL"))
 (segment (start 153.75 75.5) (end 153.75 77.25) (width 0.2) (layer "F.Cu") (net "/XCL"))
 (via (at 153.75 75.5) (size 0.6) (drill 0.3) (layers "F.Cu" "B.Cu") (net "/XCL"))
 (segment (start 153.09 71.5) (end 153.09 74.84) (width 0.2) (layer "B.Cu") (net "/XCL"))
 (segment (start 153.09 74.84) (end 153.75 75.5) (width 0.2) (layer "B.Cu") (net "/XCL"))
 (segment (start 159.475 75.425) (end 159.75 75.425) (width 0.2) (layer "F.Cu") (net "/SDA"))
 (segment (start 157.45 77.45) (end 159.475 75.425) (width 0.2) (layer "F.Cu") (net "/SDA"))
 (via (at 159.75 75.425) (size 0.6) (drill 0.3) (layers "F.Cu" "B.Cu") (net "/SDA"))
 (segment (start 158.17 71.5) (end 159.75 73.08) (width 0.2) (layer "B.Cu") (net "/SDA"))
 (segment (start 159.75 73.08) (end 159.75 75.425) (width 0.2) (layer "B.Cu") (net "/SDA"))
 (segment (start 155 75.25) (end 154.25 76) (width 0.2) (layer "F.Cu") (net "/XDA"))
 (segment (start 154.25 76) (end 154.25 76.75) (width 0.2) (layer "F.Cu") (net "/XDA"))
 (via (at 155 75.25) (size 0.6) (drill 0.3) (layers "F.Cu" "B.Cu") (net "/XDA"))
 (segment (start 155.63 74.62) (end 155 75.25) (width 0.2) (layer "B.Cu") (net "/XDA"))
 (segment (start 155.63 71.5) (end 155.63 74.62) (width 0.2) (layer "B.Cu") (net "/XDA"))
 (segment (start 151.575 85.5) (end 147.25 85.5) (width 0.2) (layer "F.Cu") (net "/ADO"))
 (segment (start 152 78) (end 152.45 78.45) (width 0.2) (layer "F.Cu") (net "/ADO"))
 (segment (start 149.975 80.612648) (end 149.975 79.026304) (width 0.2) (layer "F.Cu") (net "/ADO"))
 (segment (start 152.45 78.45) (end 153.55 78.45) (width 0.2) (layer "F.Cu") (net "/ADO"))
 (segment (start 147.25 85.5) (end 146.980779 85.230779) (width 0.2) (layer "F.Cu") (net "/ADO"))
 (segment (start 153.325 83.75) (end 153.325 83.575) (width 0.2) (layer "F.Cu") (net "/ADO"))
 (segment (start 149.975 79.026304) (end 150.276304 78.725) (width 0.2) (layer "F.Cu") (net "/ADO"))
 (segment (start 146.980779 85.230779) (end 146.980779 82.631573) (width 0.2) (layer "F.Cu") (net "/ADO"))
 (segment (start 152 76.25) (end 152 78) (width 0.2) (layer "F.Cu") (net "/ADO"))
 (segment (start 153.325 83.75) (end 151.575 85.5) (width 0.2) (layer "F.Cu") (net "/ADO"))
 (segment (start 146.980779 82.631573) (end 147.956075 82.631573) (width 0.2) (layer "F.Cu") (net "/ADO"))
 (segment (start 151.275 78.725) (end 152 78) (width 0.2) (layer "F.Cu") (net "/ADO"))
 (segment (start 152.5 75.75) (end 152 76.25) (width 0.2) (layer "F.Cu") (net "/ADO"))
 (segment (start 147.956075 82.631573) (end 149.975 80.612648) (width 0.2) (layer "F.Cu") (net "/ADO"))
 (segment (start 150.276304 78.725) (end 151.275 78.725) (width 0.2) (layer "F.Cu") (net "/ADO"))
 (via (at 152.5 75.75) (size 0.6) (drill 0.3) (layers "F.Cu" "B.Cu") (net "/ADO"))
 (segment (start 152.5 73.45) (end 152.5 75.75) (width 0.2) (layer "B.Cu") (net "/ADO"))
 (segment (start 150.55 71.5) (end 152.5 73.45) (width 0.2) (layer "B.Cu") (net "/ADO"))
 (segment (start 162.25 80.175) (end 162.25 78.75) (width 0.2) (layer "F.Cu") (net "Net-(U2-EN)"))
 (via (at 164.3 77.6125) (size 0.6) (drill 0.3) (layers "F.Cu" "B.Cu") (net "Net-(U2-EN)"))
 (via (at 162.25 78.75) (size 0.6) (drill 0.3) (layers "F.Cu" "B.Cu") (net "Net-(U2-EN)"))
 (segment (start 162.25 78.75) (end 163.1625 78.75) (width 0.2) (layer "B.Cu") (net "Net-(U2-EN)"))
 (segment (start 163.1625 78.75) (end 164.3 77.6125) (width 0.2) (layer "B.Cu") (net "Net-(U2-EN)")))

